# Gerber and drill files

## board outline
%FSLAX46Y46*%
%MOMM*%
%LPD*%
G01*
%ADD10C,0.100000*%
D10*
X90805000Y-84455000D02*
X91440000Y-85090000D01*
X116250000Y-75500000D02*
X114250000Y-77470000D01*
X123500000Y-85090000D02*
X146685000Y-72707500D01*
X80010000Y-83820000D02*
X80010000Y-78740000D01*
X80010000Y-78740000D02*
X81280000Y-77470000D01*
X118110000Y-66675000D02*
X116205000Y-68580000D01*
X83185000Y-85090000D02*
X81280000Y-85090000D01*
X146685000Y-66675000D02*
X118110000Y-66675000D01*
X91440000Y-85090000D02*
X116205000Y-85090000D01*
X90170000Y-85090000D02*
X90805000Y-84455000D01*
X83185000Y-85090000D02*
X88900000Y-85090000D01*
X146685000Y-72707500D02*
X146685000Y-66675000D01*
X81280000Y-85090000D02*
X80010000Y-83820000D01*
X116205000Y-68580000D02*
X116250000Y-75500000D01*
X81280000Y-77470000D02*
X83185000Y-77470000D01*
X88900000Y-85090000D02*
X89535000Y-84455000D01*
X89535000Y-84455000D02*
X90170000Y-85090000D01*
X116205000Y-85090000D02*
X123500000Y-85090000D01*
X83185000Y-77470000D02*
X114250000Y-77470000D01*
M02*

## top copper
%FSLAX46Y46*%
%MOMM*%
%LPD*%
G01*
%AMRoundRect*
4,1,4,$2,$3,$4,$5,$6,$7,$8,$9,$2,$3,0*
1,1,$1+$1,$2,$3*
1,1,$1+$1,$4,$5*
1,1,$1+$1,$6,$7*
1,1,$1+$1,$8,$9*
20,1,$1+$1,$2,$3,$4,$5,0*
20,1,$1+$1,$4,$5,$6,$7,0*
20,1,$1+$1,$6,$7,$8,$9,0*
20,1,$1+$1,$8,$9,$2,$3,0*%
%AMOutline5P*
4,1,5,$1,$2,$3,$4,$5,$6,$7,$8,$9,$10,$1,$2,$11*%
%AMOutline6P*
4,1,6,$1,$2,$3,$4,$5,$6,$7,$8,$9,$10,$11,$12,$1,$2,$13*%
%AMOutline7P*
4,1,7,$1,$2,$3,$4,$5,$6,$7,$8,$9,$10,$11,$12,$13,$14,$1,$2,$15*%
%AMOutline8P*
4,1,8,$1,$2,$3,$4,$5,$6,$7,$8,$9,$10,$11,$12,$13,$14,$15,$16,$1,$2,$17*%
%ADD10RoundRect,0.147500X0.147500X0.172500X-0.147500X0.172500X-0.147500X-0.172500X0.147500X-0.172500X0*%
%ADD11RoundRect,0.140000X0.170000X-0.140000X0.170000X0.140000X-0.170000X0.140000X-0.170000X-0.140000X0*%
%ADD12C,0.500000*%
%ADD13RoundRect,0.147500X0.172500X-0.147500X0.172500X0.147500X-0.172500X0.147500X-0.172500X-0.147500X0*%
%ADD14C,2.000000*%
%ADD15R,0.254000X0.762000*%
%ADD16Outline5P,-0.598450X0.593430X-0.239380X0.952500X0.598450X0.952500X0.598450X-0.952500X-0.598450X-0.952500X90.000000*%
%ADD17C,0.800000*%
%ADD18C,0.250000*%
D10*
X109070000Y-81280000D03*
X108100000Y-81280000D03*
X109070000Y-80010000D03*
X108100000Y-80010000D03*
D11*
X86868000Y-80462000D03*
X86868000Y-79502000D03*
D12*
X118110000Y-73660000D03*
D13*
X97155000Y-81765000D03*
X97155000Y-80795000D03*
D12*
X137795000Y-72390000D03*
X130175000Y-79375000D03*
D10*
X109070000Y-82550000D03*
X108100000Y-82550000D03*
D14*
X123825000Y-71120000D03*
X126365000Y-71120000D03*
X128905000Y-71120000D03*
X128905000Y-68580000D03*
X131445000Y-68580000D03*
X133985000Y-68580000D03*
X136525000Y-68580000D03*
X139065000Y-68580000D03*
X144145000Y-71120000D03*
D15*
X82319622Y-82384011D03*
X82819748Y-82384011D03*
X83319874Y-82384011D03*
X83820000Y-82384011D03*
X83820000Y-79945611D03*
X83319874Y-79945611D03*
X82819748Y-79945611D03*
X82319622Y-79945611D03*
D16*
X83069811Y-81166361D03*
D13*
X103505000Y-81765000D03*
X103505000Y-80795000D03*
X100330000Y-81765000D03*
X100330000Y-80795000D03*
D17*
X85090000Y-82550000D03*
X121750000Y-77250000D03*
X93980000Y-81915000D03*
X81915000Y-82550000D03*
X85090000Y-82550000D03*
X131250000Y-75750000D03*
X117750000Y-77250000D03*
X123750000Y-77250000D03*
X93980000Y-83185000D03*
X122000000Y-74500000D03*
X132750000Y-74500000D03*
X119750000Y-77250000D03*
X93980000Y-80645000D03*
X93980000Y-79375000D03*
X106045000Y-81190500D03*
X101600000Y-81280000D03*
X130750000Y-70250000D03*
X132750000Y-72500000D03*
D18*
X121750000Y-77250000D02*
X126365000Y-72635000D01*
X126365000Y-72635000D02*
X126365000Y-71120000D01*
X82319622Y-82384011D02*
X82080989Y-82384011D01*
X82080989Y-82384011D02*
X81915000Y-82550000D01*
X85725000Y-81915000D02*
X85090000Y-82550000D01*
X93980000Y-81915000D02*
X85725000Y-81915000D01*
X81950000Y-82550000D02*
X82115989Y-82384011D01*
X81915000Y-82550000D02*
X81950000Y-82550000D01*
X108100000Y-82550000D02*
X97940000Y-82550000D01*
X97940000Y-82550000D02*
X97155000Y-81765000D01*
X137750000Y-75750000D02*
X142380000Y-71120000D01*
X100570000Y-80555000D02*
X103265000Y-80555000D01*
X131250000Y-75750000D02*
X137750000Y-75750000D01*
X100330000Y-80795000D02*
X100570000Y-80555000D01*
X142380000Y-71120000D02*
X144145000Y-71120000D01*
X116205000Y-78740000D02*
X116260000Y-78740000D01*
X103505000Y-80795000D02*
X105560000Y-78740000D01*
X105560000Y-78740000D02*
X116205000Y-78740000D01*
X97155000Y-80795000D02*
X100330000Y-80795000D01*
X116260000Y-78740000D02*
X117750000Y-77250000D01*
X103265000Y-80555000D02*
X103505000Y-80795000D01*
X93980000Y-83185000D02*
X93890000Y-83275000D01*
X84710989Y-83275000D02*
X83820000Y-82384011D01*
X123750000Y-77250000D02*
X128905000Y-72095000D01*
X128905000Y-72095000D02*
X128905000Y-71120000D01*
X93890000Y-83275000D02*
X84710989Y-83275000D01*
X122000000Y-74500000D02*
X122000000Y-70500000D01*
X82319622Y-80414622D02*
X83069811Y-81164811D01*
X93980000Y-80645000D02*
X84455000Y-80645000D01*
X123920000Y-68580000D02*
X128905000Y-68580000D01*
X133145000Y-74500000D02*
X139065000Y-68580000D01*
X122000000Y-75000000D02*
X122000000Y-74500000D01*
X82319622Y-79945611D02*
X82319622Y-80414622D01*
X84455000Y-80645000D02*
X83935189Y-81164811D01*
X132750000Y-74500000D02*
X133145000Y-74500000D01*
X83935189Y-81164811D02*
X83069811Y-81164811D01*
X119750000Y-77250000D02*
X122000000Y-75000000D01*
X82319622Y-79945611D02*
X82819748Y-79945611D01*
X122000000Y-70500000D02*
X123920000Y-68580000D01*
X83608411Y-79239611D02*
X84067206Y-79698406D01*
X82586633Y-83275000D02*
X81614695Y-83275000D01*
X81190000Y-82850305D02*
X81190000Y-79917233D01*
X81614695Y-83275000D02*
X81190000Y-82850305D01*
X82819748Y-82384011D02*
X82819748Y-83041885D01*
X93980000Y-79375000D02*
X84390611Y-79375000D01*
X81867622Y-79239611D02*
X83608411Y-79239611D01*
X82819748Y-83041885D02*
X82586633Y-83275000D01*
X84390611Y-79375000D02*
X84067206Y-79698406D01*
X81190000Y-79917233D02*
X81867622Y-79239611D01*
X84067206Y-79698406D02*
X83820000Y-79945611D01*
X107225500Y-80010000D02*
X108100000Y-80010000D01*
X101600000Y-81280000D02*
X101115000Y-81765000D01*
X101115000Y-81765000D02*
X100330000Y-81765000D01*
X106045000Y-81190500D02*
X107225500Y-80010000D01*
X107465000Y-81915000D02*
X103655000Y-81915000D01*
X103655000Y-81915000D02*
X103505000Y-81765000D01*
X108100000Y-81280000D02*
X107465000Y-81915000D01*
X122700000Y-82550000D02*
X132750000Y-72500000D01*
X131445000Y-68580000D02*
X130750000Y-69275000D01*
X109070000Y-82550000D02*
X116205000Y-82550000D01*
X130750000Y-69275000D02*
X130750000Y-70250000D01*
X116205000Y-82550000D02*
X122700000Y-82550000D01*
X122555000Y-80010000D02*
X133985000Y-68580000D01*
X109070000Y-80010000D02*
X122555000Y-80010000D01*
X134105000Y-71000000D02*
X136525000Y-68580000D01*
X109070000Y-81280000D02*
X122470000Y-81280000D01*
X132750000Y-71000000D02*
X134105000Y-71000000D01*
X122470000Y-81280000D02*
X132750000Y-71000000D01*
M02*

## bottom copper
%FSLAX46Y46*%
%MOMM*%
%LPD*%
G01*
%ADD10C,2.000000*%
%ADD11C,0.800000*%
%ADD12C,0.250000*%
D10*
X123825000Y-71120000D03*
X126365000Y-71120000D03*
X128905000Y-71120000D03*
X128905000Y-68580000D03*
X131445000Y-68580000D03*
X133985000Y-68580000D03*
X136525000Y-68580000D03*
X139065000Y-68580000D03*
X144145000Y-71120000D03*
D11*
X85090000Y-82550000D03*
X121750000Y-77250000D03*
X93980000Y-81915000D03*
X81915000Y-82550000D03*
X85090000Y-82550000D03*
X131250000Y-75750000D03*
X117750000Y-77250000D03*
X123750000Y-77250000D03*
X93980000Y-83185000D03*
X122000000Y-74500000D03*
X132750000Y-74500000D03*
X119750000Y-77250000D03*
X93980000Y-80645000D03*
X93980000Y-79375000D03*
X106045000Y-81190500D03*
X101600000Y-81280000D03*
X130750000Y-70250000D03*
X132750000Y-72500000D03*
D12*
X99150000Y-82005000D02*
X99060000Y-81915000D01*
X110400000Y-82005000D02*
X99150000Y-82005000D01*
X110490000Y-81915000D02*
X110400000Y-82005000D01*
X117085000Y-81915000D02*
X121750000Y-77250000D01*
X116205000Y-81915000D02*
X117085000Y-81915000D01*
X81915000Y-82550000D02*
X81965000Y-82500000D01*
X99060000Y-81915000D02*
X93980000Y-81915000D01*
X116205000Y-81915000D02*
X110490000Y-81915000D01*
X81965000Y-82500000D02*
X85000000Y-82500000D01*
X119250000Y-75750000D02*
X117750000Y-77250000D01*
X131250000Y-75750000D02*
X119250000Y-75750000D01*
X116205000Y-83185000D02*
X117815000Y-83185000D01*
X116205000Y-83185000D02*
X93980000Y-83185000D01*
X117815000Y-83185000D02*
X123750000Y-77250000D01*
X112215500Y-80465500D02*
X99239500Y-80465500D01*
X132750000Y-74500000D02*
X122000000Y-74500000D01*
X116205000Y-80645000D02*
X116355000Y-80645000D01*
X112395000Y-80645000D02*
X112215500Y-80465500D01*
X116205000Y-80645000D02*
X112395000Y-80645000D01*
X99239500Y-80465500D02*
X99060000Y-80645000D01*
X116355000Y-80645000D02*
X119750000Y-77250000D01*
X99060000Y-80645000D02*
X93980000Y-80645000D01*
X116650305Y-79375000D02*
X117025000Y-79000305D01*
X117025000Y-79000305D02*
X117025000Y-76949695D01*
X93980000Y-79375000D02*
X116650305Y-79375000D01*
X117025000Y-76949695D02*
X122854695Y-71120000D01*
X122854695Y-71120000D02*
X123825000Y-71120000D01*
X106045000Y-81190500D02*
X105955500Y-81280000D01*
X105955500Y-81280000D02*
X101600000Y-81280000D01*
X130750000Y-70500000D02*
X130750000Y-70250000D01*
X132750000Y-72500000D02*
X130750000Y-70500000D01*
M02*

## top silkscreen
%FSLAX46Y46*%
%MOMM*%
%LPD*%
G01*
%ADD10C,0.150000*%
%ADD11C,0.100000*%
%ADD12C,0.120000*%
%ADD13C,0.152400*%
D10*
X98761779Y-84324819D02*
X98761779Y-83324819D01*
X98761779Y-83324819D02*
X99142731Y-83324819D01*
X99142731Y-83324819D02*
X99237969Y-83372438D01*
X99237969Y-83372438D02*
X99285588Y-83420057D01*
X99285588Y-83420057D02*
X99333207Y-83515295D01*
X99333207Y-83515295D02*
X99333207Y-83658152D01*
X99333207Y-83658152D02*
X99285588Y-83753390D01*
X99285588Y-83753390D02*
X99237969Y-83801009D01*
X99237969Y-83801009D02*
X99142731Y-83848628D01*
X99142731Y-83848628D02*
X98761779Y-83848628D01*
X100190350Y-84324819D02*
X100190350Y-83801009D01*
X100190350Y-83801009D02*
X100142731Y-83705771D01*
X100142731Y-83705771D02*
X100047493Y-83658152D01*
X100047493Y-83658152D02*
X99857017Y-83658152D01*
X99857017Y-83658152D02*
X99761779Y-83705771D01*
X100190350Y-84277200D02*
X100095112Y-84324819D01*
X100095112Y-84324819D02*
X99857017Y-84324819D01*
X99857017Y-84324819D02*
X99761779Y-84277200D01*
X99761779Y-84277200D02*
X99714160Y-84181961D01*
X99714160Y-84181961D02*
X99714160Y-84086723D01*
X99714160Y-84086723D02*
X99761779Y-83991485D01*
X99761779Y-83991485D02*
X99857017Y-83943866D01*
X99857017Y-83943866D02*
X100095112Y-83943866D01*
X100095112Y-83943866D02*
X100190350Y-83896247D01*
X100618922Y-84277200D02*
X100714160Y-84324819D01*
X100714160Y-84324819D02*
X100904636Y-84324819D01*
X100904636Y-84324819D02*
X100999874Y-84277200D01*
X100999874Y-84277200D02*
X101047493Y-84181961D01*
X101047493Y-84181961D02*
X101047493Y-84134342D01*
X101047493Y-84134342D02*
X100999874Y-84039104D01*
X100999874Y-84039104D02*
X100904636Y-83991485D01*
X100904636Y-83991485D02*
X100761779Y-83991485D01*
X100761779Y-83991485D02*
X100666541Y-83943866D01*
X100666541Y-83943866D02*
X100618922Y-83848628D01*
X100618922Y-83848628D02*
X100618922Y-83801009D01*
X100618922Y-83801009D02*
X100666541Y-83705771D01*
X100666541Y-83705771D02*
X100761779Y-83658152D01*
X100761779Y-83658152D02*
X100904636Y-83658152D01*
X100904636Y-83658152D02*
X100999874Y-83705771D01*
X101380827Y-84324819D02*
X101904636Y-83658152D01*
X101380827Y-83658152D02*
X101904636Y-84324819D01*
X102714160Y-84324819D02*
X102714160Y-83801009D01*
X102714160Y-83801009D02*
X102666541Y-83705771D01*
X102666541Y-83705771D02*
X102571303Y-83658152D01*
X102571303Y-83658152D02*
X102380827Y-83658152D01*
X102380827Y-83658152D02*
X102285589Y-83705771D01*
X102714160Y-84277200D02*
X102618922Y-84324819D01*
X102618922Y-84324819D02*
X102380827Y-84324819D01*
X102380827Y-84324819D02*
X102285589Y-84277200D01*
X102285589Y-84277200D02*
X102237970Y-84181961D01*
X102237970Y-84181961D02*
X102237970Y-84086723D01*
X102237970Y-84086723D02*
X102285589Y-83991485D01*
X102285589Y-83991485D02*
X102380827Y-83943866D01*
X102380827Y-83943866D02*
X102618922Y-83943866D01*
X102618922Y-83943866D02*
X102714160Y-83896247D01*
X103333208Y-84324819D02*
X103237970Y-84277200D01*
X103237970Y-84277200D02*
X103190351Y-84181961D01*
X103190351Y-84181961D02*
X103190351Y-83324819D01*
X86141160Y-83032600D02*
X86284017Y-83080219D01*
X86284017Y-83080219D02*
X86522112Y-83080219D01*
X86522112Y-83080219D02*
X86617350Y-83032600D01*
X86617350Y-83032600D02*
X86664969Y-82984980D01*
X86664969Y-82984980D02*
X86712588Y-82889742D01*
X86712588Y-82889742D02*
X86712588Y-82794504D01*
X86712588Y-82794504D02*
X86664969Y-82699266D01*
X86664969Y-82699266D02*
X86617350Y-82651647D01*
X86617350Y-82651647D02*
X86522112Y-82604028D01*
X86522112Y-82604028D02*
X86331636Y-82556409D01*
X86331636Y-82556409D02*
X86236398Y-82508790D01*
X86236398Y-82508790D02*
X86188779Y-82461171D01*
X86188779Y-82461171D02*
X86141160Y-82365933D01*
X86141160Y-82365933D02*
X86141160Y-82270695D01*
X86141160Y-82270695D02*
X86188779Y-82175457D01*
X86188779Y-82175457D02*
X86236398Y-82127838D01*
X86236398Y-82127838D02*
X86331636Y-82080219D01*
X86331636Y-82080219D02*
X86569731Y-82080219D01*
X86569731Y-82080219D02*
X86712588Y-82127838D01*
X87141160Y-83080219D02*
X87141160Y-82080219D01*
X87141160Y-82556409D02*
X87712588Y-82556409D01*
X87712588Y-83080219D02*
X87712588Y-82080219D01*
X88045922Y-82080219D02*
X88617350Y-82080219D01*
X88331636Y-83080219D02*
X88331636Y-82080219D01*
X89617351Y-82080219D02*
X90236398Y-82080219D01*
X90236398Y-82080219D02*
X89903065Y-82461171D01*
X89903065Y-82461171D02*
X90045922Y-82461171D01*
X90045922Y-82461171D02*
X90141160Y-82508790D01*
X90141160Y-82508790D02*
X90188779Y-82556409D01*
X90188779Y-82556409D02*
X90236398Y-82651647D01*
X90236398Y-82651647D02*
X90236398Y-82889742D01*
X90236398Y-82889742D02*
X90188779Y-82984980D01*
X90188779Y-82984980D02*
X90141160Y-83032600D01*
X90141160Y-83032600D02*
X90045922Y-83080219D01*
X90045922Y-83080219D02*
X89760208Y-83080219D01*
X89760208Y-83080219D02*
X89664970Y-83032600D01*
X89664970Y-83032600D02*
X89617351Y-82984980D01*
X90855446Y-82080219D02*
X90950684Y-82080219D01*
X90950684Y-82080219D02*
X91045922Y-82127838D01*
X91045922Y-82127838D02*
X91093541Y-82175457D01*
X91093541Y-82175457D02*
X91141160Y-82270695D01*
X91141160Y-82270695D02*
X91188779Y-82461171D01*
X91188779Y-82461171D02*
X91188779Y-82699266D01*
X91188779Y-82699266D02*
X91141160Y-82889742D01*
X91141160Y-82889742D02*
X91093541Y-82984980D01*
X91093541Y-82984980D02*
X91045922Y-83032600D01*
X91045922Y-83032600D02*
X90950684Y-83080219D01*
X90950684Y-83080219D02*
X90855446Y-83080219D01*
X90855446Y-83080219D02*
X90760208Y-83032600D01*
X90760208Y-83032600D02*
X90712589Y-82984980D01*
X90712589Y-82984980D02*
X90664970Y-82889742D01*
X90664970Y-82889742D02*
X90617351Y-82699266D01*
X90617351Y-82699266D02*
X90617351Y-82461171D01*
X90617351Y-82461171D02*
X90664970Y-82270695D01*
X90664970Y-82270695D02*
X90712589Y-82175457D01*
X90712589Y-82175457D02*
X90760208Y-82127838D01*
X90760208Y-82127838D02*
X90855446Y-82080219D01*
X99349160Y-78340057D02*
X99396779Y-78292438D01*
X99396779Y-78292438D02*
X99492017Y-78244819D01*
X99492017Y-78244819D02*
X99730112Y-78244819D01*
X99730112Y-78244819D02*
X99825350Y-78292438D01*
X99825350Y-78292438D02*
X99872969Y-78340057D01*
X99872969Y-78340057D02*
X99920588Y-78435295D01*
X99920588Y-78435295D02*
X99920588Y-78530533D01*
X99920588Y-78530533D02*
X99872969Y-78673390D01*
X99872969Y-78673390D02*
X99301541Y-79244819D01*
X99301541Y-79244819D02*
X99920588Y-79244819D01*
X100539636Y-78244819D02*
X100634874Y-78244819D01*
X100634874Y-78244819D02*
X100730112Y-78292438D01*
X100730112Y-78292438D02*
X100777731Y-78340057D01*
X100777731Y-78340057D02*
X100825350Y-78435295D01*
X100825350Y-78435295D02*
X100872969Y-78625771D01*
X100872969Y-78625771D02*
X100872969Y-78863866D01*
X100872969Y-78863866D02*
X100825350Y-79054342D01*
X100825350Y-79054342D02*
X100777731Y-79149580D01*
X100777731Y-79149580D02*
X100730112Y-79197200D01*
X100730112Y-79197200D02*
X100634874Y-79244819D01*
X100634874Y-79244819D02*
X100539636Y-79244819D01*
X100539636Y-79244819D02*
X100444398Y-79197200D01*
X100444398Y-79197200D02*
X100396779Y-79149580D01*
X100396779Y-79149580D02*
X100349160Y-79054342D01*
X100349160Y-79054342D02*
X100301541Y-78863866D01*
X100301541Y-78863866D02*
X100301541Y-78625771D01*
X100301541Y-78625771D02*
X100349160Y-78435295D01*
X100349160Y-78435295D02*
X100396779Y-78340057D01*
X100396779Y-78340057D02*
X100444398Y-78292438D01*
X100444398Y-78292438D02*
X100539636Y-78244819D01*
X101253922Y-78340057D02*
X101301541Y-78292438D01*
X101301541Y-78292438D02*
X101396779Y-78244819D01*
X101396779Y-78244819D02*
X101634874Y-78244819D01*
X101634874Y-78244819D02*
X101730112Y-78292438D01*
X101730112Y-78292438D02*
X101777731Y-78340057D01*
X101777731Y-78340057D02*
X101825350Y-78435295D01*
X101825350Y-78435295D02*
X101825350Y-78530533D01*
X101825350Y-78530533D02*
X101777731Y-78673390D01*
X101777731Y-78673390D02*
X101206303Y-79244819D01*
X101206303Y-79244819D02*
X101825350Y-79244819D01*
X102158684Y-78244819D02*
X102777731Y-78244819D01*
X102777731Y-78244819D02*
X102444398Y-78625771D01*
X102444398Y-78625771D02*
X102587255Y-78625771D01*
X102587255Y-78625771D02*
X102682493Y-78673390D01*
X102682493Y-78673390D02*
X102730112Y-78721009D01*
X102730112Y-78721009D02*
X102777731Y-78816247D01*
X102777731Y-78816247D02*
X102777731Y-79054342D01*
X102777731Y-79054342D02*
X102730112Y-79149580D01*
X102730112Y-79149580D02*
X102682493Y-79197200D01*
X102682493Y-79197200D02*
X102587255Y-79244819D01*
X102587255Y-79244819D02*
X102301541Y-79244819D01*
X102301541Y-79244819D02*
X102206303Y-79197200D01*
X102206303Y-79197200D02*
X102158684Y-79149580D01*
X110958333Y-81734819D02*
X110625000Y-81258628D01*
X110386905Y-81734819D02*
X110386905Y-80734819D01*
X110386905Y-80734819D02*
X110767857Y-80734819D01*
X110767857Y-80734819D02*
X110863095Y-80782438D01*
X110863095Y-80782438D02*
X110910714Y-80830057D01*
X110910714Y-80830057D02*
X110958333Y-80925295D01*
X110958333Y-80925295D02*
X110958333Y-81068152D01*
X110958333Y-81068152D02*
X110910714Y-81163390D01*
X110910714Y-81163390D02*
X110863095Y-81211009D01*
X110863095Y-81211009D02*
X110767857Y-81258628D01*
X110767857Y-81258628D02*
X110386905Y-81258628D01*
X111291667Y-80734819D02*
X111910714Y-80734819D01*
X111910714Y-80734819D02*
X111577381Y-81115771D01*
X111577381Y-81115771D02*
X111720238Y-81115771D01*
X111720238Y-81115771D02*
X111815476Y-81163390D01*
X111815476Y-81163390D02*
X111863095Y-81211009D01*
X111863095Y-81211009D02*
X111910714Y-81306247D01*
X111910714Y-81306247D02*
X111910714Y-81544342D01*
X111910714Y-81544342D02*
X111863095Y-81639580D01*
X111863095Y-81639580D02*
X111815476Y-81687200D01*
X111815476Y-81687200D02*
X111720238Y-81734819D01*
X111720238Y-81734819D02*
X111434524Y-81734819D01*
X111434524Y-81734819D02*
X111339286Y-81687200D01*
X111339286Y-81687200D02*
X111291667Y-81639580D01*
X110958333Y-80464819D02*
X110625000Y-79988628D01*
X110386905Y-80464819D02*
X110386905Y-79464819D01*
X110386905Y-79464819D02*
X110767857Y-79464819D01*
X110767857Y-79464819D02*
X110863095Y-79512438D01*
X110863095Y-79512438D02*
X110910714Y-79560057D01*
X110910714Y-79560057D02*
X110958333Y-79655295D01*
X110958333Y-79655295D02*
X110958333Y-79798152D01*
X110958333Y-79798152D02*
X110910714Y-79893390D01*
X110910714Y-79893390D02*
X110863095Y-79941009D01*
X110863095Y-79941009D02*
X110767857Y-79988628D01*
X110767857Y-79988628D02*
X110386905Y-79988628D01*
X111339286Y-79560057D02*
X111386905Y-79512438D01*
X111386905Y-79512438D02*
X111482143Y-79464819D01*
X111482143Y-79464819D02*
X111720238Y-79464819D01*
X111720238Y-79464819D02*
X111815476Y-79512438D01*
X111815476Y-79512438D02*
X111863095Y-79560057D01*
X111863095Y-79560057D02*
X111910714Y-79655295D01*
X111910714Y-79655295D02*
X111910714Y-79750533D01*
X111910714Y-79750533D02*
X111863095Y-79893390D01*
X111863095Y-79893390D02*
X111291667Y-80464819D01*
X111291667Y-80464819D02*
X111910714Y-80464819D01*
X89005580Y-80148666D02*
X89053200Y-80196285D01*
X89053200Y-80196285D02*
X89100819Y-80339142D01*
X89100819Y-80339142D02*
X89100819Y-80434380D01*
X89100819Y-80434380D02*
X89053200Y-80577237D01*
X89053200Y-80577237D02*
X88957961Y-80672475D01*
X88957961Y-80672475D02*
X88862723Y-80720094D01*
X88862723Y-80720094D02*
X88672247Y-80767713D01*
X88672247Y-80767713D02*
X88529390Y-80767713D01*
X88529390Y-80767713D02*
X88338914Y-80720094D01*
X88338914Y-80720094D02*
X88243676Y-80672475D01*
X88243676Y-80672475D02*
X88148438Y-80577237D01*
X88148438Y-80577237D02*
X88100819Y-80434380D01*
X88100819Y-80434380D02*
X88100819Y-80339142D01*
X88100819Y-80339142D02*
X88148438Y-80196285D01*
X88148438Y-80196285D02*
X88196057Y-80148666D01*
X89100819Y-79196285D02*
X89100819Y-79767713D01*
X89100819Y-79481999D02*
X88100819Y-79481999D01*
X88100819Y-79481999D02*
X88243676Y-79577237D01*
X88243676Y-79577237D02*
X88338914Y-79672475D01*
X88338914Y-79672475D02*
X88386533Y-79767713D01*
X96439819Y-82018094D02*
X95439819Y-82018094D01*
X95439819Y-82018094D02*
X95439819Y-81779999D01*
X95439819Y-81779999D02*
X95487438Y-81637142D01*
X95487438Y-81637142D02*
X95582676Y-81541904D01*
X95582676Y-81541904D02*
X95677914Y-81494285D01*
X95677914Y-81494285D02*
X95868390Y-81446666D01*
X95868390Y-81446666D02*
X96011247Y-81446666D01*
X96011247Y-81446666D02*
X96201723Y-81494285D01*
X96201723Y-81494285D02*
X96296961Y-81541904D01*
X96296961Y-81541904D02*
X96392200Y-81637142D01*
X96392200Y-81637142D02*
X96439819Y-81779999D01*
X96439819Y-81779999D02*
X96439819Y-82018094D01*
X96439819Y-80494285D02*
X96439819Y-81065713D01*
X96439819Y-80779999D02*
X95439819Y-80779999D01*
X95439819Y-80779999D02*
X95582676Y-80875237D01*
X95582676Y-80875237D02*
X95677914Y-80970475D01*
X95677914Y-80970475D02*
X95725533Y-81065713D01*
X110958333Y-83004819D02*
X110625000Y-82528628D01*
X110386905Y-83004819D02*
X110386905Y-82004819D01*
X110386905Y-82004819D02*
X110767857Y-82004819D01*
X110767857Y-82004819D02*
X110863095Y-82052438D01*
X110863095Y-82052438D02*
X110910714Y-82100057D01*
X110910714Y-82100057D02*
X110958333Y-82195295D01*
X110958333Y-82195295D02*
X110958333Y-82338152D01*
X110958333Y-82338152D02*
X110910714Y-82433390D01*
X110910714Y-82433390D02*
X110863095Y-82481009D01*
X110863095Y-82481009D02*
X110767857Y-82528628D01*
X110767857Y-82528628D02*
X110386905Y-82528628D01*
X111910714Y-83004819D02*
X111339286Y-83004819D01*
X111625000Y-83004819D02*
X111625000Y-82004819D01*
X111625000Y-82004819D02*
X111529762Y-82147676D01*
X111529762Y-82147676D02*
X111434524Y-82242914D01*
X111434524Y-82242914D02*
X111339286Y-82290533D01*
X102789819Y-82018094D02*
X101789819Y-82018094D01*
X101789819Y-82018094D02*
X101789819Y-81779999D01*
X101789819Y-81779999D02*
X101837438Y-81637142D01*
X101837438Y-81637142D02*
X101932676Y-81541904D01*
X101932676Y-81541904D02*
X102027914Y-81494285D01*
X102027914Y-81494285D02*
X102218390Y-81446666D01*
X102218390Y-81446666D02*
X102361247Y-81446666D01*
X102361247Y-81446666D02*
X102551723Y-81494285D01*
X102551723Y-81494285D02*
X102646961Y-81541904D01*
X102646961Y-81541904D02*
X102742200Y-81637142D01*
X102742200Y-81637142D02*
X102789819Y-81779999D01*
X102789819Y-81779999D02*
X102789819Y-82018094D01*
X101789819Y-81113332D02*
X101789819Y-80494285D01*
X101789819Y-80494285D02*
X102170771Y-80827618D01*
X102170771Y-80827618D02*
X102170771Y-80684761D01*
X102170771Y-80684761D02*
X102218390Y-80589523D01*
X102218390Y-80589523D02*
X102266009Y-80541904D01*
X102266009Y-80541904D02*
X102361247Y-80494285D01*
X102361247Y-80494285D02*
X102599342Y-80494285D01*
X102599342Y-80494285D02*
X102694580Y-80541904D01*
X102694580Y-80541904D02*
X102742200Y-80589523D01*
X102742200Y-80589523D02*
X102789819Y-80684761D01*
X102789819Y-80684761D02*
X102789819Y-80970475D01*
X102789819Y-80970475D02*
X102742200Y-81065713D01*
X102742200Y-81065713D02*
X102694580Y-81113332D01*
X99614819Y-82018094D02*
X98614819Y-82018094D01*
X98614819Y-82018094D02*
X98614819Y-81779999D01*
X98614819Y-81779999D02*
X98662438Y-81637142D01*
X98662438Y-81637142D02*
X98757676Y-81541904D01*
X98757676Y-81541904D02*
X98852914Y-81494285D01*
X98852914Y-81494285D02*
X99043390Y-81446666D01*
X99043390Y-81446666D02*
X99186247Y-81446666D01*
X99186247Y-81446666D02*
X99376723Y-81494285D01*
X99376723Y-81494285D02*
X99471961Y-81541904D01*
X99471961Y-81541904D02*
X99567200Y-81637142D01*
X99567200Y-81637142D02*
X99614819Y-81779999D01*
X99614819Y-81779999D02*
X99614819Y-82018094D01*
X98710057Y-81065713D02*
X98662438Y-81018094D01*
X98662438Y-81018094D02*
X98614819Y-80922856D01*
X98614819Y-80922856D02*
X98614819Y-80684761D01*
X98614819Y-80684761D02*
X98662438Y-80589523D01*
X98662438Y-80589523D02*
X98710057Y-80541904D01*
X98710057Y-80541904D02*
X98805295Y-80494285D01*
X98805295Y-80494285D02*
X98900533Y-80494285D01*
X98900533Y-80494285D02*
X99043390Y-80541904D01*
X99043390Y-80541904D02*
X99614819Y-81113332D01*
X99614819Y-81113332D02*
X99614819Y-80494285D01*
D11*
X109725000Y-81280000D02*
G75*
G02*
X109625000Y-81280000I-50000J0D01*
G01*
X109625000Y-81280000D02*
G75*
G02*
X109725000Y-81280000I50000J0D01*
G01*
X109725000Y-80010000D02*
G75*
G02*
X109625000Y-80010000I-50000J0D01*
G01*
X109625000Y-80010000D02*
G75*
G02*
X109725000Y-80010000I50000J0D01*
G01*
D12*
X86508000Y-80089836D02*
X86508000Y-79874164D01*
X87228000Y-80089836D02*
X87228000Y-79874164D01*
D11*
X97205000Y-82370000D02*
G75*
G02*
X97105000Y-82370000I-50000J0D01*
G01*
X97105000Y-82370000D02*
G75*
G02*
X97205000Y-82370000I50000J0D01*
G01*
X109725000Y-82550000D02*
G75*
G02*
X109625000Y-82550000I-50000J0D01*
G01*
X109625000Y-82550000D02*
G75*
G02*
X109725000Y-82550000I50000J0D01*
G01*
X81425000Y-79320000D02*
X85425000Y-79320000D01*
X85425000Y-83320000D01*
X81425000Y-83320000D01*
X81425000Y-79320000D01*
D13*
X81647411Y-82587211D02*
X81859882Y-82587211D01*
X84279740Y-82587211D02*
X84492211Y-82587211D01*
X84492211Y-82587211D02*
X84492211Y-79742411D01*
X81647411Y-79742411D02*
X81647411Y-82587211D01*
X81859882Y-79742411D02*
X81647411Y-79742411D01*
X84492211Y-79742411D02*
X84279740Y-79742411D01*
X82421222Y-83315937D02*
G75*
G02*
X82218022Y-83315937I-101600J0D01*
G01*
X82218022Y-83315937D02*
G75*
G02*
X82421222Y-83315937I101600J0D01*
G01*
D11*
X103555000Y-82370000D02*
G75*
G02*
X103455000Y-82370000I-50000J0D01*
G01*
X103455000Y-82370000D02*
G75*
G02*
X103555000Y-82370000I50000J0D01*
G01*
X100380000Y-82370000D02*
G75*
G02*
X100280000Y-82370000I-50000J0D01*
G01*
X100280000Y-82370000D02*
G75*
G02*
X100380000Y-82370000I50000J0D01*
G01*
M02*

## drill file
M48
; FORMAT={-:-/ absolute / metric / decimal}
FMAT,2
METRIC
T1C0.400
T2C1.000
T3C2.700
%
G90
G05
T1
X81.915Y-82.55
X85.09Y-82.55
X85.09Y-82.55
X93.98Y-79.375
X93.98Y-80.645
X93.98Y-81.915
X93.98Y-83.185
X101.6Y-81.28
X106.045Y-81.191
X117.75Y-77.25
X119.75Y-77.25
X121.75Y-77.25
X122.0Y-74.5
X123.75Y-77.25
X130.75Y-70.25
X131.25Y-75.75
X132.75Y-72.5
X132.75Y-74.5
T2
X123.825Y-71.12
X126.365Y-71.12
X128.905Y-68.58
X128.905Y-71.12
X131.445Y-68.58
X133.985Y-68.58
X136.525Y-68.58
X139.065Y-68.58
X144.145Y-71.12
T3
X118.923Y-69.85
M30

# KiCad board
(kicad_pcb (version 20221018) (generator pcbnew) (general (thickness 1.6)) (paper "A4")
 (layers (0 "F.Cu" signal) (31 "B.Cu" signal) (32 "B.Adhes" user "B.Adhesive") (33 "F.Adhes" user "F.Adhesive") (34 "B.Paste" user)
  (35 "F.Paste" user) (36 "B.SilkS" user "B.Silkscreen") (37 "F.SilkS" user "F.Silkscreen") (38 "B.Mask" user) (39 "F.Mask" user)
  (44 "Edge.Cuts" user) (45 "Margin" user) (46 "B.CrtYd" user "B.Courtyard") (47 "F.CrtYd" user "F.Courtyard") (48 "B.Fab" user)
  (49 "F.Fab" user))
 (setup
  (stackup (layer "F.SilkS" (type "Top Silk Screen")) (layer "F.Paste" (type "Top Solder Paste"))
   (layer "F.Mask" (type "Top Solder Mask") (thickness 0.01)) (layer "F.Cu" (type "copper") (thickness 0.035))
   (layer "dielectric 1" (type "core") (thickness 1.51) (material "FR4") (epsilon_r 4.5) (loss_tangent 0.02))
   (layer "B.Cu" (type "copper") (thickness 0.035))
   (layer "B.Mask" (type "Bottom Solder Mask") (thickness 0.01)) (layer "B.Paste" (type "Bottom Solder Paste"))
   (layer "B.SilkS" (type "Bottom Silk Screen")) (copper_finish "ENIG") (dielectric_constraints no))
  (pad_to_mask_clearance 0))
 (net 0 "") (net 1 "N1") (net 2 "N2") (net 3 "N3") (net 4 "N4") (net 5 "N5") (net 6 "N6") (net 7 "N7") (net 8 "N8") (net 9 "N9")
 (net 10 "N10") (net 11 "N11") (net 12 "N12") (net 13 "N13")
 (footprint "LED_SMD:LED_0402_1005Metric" (layer "F.Cu") (at 108.585 81.28 180)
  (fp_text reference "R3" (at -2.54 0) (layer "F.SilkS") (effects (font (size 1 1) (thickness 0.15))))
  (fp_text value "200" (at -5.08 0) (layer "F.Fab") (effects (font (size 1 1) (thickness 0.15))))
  (fp_circle (center -1.09 0) (end -1.04 0) (stroke (width 0.1) (type solid)) (fill none) (layer "F.SilkS"))
  (pad "1" smd roundrect (at -0.485 0 180) (size 0.59 0.64) (layers "F.Cu" "F.Paste" "F.Mask") (roundrect_rratio 0.25) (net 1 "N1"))
  (pad "2" smd roundrect (at 0.485 0 180) (size 0.59 0.64) (layers "F.Cu" "F.Paste" "F.Mask") (roundrect_rratio 0.25) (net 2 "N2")))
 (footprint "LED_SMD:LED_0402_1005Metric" (layer "F.Cu") (at 108.585 80.01 180)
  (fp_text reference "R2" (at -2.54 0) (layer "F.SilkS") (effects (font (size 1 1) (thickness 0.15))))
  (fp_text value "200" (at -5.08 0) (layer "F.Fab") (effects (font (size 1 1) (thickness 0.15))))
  (fp_circle (center -1.09 0) (end -1.04 0) (stroke (width 0.1) (type solid)) (fill none) (layer "F.SilkS"))
  (pad "1" smd roundrect (at -0.485 0 180) (size 0.59 0.64) (layers "F.Cu" "F.Paste" "F.Mask") (roundrect_rratio 0.25) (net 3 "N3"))
  (pad "2" smd roundrect (at 0.485 0 180) (size 0.59 0.64) (layers "F.Cu" "F.Paste" "F.Mask") (roundrect_rratio 0.25) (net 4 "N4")))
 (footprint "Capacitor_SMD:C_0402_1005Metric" (layer "F.Cu") (at 86.868 79.982 90)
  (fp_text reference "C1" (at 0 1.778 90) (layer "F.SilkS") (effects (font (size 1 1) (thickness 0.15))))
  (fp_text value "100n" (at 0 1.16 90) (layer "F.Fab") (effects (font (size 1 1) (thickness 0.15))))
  (fp_line (start -0.107836 -0.36) (end 0.107836 -0.36) (stroke (width 0.12) (type solid)) (layer "F.SilkS"))
  (fp_line (start -0.107836 0.36) (end 0.107836 0.36) (stroke (width 0.12) (type solid)) (layer "F.SilkS"))
  (pad "1" smd roundrect (at -0.48 0 90) (size 0.56 0.62) (layers "F.Cu" "F.Paste" "F.Mask") (roundrect_rratio 0.25) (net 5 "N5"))
  (pad "2" smd roundrect (at 0.48 0 90) (size 0.56 0.62) (layers "F.Cu" "F.Paste" "F.Mask") (roundrect_rratio 0.25) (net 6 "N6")))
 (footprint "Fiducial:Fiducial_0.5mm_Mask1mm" (layer "F.Cu") (at 118.11 73.66)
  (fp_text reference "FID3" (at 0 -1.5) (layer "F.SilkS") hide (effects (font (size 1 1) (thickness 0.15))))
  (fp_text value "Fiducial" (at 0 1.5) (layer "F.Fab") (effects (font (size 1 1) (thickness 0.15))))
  (pad "" smd circle (at 0 0) (size 0.5 0.5) (layers "F.Cu" "F.Mask") (solder_mask_margin 0.25) (clearance 0.25)))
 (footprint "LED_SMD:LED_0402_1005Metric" (layer "F.Cu") (at 97.155 81.28 90)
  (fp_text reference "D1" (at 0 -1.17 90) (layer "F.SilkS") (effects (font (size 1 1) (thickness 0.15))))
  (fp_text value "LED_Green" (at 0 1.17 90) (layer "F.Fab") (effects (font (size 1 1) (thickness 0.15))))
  (fp_circle (center -1.09 0) (end -1.04 0) (stroke (width 0.1) (type solid)) (fill none) (layer "F.SilkS"))
  (pad "1" smd roundrect (at -0.485 0 90) (size 0.59 0.64) (layers "F.Cu" "F.Paste" "F.Mask") (roundrect_rratio 0.25) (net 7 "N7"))
  (pad "2" smd roundrect (at 0.485 0 90) (size 0.59 0.64) (layers "F.Cu" "F.Paste" "F.Mask") (roundrect_rratio 0.25) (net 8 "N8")))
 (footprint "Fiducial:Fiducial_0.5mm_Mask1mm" (layer "F.Cu") (at 137.795 72.39)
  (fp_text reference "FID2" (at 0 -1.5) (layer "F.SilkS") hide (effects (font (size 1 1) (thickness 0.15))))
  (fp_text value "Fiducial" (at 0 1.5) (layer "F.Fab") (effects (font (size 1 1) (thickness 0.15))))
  (pad "" smd circle (at 0 0) (size 0.5 0.5) (layers "F.Cu" "F.Mask") (solder_mask_margin 0.25) (clearance 0.25)))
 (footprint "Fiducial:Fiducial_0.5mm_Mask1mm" (layer "F.Cu") (at 130.175 79.375)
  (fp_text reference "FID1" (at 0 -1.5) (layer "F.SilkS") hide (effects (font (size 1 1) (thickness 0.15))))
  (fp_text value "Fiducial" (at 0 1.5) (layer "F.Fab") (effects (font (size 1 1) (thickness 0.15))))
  (pad "" smd circle (at 0 0) (size 0.5 0.5) (layers "F.Cu" "F.Mask") (solder_mask_margin 0.25) (clearance 0.25)))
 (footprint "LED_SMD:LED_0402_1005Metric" (layer "F.Cu") (at 108.585 82.55 180)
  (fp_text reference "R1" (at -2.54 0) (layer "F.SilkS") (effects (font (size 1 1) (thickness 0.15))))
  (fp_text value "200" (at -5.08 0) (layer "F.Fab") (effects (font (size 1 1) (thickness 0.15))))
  (fp_circle (center -1.09 0) (end -1.04 0) (stroke (width 0.1) (type solid)) (fill none) (layer "F.SilkS"))
  (pad "1" smd roundrect (at -0.485 0 180) (size 0.59 0.64) (layers "F.Cu" "F.Paste" "F.Mask") (roundrect_rratio 0.25) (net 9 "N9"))
  (pad "2" smd roundrect (at 0.485 0 180) (size 0.59 0.64) (layers "F.Cu" "F.Paste" "F.Mask") (roundrect_rratio 0.25) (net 7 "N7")))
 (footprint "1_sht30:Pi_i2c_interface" (layer "F.Cu") (at 123.825 71.12)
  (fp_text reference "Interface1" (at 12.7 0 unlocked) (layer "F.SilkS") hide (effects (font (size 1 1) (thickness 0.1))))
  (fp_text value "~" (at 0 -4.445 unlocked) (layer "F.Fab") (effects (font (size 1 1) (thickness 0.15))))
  (fp_rect (start -42.4 8.2) (end -38.4 12.2) (stroke (width 0.1) (type default)) (fill none) (layer "F.SilkS"))
  (pad "1" thru_hole circle (at 0 0) (size 2 2) (drill 1) (layers "*.Cu" "*.Mask") (remove_unused_layers) (keep_end_layers)
   (zone_layer_connections) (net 6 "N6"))
  (pad "2" thru_hole circle (at 2.54 0) (size 2 2) (drill 1) (layers "*.Cu" "*.Mask") (remove_unused_layers) (keep_end_layers)
   (zone_layer_connections) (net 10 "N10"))
  (pad "3" thru_hole circle (at 5.08 0) (size 2 2) (drill 1) (layers "*.Cu" "*.Mask") (remove_unused_layers) (keep_end_layers)
   (zone_layer_connections) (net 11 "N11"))
  (pad "4" thru_hole circle (at 5.08 -2.54) (size 2 2) (drill 1) (layers "*.Cu" "*.Mask") (remove_unused_layers) (keep_end_layers)
   (zone_layer_connections) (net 5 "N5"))
  (pad "5" thru_hole circle (at 7.62 -2.54) (size 2 2) (drill 1) (layers "*.Cu" "*.Mask") (remove_unused_layers) (keep_end_layers)
   (zone_layer_connections) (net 9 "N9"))
  (pad "6" thru_hole circle (at 10.16 -2.54) (size 2 2) (drill 1) (layers "*.Cu" "*.Mask") (remove_unused_layers) (keep_end_layers)
   (zone_layer_connections) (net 3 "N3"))
  (pad "7" thru_hole circle (at 12.7 -2.54) (size 2 2) (drill 1) (layers "*.Cu" "*.Mask") (remove_unused_layers) (keep_end_layers)
   (zone_layer_connections) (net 1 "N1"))
  (pad "8" thru_hole circle (at 15.24 -2.54) (size 2 2) (drill 1) (layers "*.Cu" "*.Mask") (remove_unused_layers) (keep_end_layers)
   (zone_layer_connections) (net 5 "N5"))
  (pad "9" thru_hole circle (at 20.32 0) (size 2 2) (drill 1) (layers "*.Cu" "*.Mask") (remove_unused_layers) (keep_end_layers)
   (zone_layer_connections) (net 8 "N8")))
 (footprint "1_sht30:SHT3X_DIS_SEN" (layer "F.Cu") (at 83.069811 81.164811 90)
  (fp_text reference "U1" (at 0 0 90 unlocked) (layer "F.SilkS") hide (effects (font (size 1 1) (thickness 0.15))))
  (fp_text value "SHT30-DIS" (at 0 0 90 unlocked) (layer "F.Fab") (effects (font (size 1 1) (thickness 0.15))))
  (fp_line (start -1.4224 -1.4224) (end -1.4224 -1.209929) (stroke (width 0.1524) (type solid)) (layer "F.SilkS"))
  (fp_line (start -1.4224 1.209929) (end -1.4224 1.4224) (stroke (width 0.1524) (type solid)) (layer "F.SilkS"))
  (fp_line (start -1.4224 1.4224) (end 1.4224 1.4224) (stroke (width 0.1524) (type solid)) (layer "F.SilkS"))
  (fp_line (start 1.4224 -1.4224) (end -1.4224 -1.4224) (stroke (width 0.1524) (type solid)) (layer "F.SilkS"))
  (fp_line (start 1.4224 -1.209929) (end 1.4224 -1.4224) (stroke (width 0.1524) (type solid)) (layer "F.SilkS"))
  (fp_line (start 1.4224 1.4224) (end 1.4224 1.209929) (stroke (width 0.1524) (type solid)) (layer "F.SilkS"))
  (fp_circle (center -2.151126 -0.750189) (end -2.049526 -0.750189) (stroke (width 0.1524) (type solid)) (fill none) (layer "F.SilkS"))
  (pad "1" smd rect (at -1.2192 -0.750189 90) (size 0.762 0.254) (layers "F.Cu" "F.Paste" "F.Mask") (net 10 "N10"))
  (pad "2" smd rect (at -1.2192 -0.250063 90) (size 0.762 0.254) (layers "F.Cu" "F.Paste" "F.Mask") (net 6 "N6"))
  (pad "3" smd rect (at -1.2192 0.250063 90) (size 0.762 0.254) (layers "F.Cu" "F.Paste" "F.Mask") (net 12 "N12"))
  (pad "4" smd rect (at -1.2192 0.750189 90) (size 0.762 0.254) (layers "F.Cu" "F.Paste" "F.Mask") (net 11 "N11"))
  (pad "5" smd rect (at 1.2192 0.750189 90) (size 0.762 0.254) (layers "F.Cu" "F.Paste" "F.Mask") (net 6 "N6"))
  (pad "6" smd rect (at 1.2192 0.250063 90) (size 0.762 0.254) (layers "F.Cu" "F.Paste" "F.Mask") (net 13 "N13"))
  (pad "7" smd rect (at 1.2192 -0.250063 90) (size 0.762 0.254) (layers "F.Cu" "F.Paste" "F.Mask") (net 5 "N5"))
  (pad "8" smd rect (at 1.2192 -0.750189 90) (size 0.762 0.254) (layers "F.Cu" "F.Paste" "F.Mask") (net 5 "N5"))
  (pad "9" smd roundrect (at -0.00155 0 90) (size 1.1969 1.905) (layers "F.Cu" "F.Paste" "F.Mask") (roundrect_rratio 0) (chamfer_ratio 0.3)
   (chamfer top_left) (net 5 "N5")))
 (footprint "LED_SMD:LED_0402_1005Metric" (layer "F.Cu") (at 103.505 81.28 90)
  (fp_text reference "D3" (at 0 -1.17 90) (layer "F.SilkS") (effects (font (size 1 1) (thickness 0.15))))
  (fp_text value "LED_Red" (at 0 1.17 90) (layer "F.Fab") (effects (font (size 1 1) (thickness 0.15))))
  (fp_circle (center -1.09 0) (end -1.04 0) (stroke (width 0.1) (type solid)) (fill none) (layer "F.SilkS"))
  (pad "1" smd roundrect (at -0.485 0 90) (size 0.59 0.64) (layers "F.Cu" "F.Paste" "F.Mask") (roundrect_rratio 0.25) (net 2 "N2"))
  (pad "2" smd roundrect (at 0.485 0 90) (size 0.59 0.64) (layers "F.Cu" "F.Paste" "F.Mask") (roundrect_rratio 0.25) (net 8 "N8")))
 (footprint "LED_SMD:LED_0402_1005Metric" (layer "F.Cu") (at 100.33 81.28 90)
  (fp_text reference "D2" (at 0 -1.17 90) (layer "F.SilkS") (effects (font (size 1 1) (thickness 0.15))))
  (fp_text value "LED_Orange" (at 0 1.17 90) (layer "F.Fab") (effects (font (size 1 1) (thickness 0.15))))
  (fp_circle (center -1.09 0) (end -1.04 0) (stroke (width 0.1) (type solid)) (fill none) (layer "F.SilkS"))
  (pad "1" smd roundrect (at -0.485 0 90) (size 0.59 0.64) (layers "F.Cu" "F.Paste" "F.Mask") (roundrect_rratio 0.25) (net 4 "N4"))
  (pad "2" smd roundrect (at 0.485 0 90) (size 0.59 0.64) (layers "F.Cu" "F.Paste" "F.Mask") (roundrect_rratio 0.25) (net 8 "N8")))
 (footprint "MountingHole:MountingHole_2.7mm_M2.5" (layer "F.Cu") (at 118.9228 69.85)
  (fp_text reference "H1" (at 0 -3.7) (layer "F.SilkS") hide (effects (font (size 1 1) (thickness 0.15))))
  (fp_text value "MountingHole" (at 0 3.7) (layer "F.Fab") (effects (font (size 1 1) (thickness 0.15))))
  (pad "" np_thru_hole circle (at 0 0) (size 2.7 2.7) (drill 2.7) (layers "*.Cu" "*.Mask")))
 (gr_line (start 90.805 84.455) (end 91.44 85.09) (stroke (width 0.1) (type default)) (layer "Edge.Cuts"))
 (gr_line (start 116.25 75.5) (end 114.25 77.47) (stroke (width 0.1) (type default)) (layer "Edge.Cuts"))
 (gr_line (start 123.5 85.09) (end 146.685 72.7075) (stroke (width 0.1) (type default)) (layer "Edge.Cuts"))
 (gr_line (start 80.01 83.82) (end 80.01 78.74) (stroke (width 0.1) (type default)) (layer "Edge.Cuts"))
 (gr_line (start 80.01 78.74) (end 81.28 77.47) (stroke (width 0.1) (type default)) (layer "Edge.Cuts"))
 (gr_line (start 118.11 66.675) (end 116.205 68.58) (stroke (width 0.1) (type default)) (layer "Edge.Cuts"))
 (gr_line (start 83.185 85.09) (end 81.28 85.09) (stroke (width 0.1) (type default)) (layer "Edge.Cuts"))
 (gr_line (start 146.685 66.675) (end 118.11 66.675) (stroke (width 0.1) (type default)) (layer "Edge.Cuts"))
 (gr_line (start 91.44 85.09) (end 116.205 85.09) (stroke (width 0.1) (type default)) (layer "Edge.Cuts"))
 (gr_line (start 90.17 85.09) (end 90.805 84.455) (stroke (width 0.1) (type default)) (layer "Edge.Cuts"))
 (gr_line (start 83.185 85.09) (end 88.9 85.09) (stroke (width 0.1) (type default)) (layer "Edge.Cuts"))
 (gr_line (start 146.685 72.7075) (end 146.685 66.675) (stroke (width 0.1) (type default)) (layer "Edge.Cuts"))
 (gr_line (start 81.28 85.09) (end 80.01 83.82) (stroke (width 0.1) (type default)) (layer "Edge.Cuts"))
 (gr_line (start 116.205 68.58) (end 116.25 75.5) (stroke (width 0.1) (type default)) (layer "Edge.Cuts"))
 (gr_line (start 81.28 77.47) (end 83.185 77.47) (stroke (width 0.1) (type default)) (layer "Edge.Cuts"))
 (gr_line (start 88.9 85.09) (end 89.535 84.455) (stroke (width 0.1) (type default)) (layer "Edge.Cuts"))
 (gr_line (start 89.535 84.455) (end 90.17 85.09) (stroke (width 0.1) (type default)) (layer "Edge.Cuts"))
 (gr_line (start 116.205 85.09) (end 123.5 85.09) (stroke (width 0.1) (type default)) (layer "Edge.Cuts"))
 (gr_line (start 83.185 77.47) (end 114.25 77.47) (stroke (width 0.1) (type default)) (layer "Edge.Cuts"))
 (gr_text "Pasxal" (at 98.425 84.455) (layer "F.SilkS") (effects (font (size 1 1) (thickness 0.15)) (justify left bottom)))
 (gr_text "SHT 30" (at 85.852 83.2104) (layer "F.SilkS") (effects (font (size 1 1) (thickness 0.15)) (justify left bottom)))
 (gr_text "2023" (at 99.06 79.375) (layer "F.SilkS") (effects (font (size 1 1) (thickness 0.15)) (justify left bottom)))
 (segment (start 121.75 77.25) (end 126.365 72.635) (width 0.25) (layer "F.Cu") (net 10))
 (segment (start 126.365 72.635) (end 126.365 71.12) (width 0.25) (layer "F.Cu") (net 10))
 (segment (start 82.319622 82.384011) (end 82.080989 82.384011) (width 0.25) (layer "F.Cu") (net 10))
 (segment (start 82.080989 82.384011) (end 81.915 82.55) (width 0.25) (layer "F.Cu") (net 10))
 (segment (start 85.725 81.915) (end 85.09 82.55) (width 0.25) (layer "F.Cu") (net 10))
 (segment (start 93.98 81.915) (end 85.725 81.915) (width 0.25) (layer "F.Cu") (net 10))
 (segment (start 81.95 82.55) (end 82.115989 82.384011) (width 0.25) (layer "F.Cu") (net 10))
 (segment (start 81.915 82.55) (end 81.95 82.55) (width 0.25) (layer "F.Cu") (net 10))
 (via (at 85.09 82.55) (size 0.8) (drill 0.4) (layers "F.Cu" "B.Cu") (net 10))
 (via (at 121.75 77.25) (size 0.8) (drill 0.4) (layers "F.Cu" "B.Cu") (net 10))
 (via (at 93.98 81.915) (size 0.8) (drill 0.4) (layers "F.Cu" "B.Cu") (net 10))
 (via (at 81.915 82.55) (size 0.8) (drill 0.4) (layers "F.Cu" "B.Cu") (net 10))
 (via (at 85.09 82.55) (size 0.8) (drill 0.4) (layers "F.Cu" "B.Cu") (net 10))
 (segment (start 99.15 82.005) (end 99.06 81.915) (width 0.25) (layer "B.Cu") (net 10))
 (segment (start 110.4 82.005) (end 99.15 82.005) (width 0.25) (layer "B.Cu") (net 10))
 (segment (start 110.49 81.915) (end 110.4 82.005) (width 0.25) (layer "B.Cu") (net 10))
 (segment (start 117.085 81.915) (end 121.75 77.25) (width 0.25) (layer "B.Cu") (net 10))
 (segment (start 116.205 81.915) (end 117.085 81.915) (width 0.25) (layer "B.Cu") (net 10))
 (segment (start 81.915 82.55) (end 81.965 82.5) (width 0.25) (layer "B.Cu") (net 10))
 (segment (start 99.06 81.915) (end 93.98 81.915) (width 0.25) (layer "B.Cu") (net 10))
 (segment (start 116.205 81.915) (end 110.49 81.915) (width 0.25) (layer "B.Cu") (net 10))
 (segment (start 81.965 82.5) (end 85 82.5) (width 0.25) (layer "B.Cu") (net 10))
 (segment (start 108.1 82.55) (end 97.94 82.55) (width 0.25) (layer "F.Cu") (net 7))
 (segment (start 97.94 82.55) (end 97.155 81.765) (width 0.25) (layer "F.Cu") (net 7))
 (segment (start 137.75 75.75) (end 142.38 71.12) (width 0.25) (layer "F.Cu") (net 8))
 (segment (start 100.57 80.555) (end 103.265 80.555) (width 0.25) (layer "F.Cu") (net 8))
 (segment (start 131.25 75.75) (end 137.75 75.75) (width 0.25) (layer "F.Cu") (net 8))
 (segment (start 100.33 80.795) (end 100.57 80.555) (width 0.25) (layer "F.Cu") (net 8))
 (segment (start 142.38 71.12) (end 144.145 71.12) (width 0.25) (layer "F.Cu") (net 8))
 (segment (start 116.205 78.74) (end 116.26 78.74) (width 0.25) (layer "F.Cu") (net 8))
 (segment (start 103.505 80.795) (end 105.56 78.74) (width 0.25) (layer "F.Cu") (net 8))
 (segment (start 105.56 78.74) (end 116.205 78.74) (width 0.25) (layer "F.Cu") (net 8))
 (segment (start 97.155 80.795) (end 100.33 80.795) (width 0.25) (layer "F.Cu") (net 8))
 (segment (start 116.26 78.74) (end 117.75 77.25) (width 0.25) (layer "F.Cu") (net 8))
 (segment (start 103.265 80.555) (end 103.505 80.795) (width 0.25) (layer "F.Cu") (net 8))
 (via (at 131.25 75.75) (size 0.8) (drill 0.4) (layers "F.Cu" "B.Cu") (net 8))
 (via (at 117.75 77.25) (size 0.8) (drill 0.4) (layers "F.Cu" "B.Cu") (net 8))
 (segment (start 119.25 75.75) (end 117.75 77.25) (width 0.25) (layer "B.Cu") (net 8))
 (segment (start 131.25 75.75) (end 119.25 75.75) (width 0.25) (layer "B.Cu") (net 8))
 (segment (start 93.98 83.185) (end 93.89 83.275) (width 0.25) (layer "F.Cu") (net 11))
 (segment (start 84.710989 83.275) (end 83.82 82.384011) (width 0.25) (layer "F.Cu") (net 11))
 (segment (start 123.75 77.25) (end 128.905 72.095) (width 0.25) (layer "F.Cu") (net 11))
 (segment (start 128.905 72.095) (end 128.905 71.12) (width 0.25) (layer "F.Cu") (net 11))
 (segment (start 93.89 83.275) (end 84.710989 83.275) (width 0.25) (layer "F.Cu") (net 11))
 (via (at 123.75 77.25) (size 0.8) (drill 0.4) (layers "F.Cu" "B.Cu") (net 11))
 (via (at 93.98 83.185) (size 0.8) (drill 0.4) (layers "F.Cu" "B.Cu") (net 11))
 (segment (start 116.205 83.185) (end 117.815 83.185) (width 0.25) (layer "B.Cu") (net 11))
 (segment (start 116.205 83.185) (end 93.98 83.185) (width 0.25) (layer "B.Cu") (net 11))
 (segment (start 117.815 83.185) (end 123.75 77.25) (width 0.25) (layer "B.Cu") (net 11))
 (segment (start 122 74.5) (end 122 70.5) (width 0.25) (layer "F.Cu") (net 5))
 (segment (start 82.319622 80.414622) (end 83.069811 81.164811) (width 0.25) (layer "F.Cu") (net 5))
 (segment (start 93.98 80.645) (end 84.455 80.645) (width 0.25) (layer "F.Cu") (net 5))
 (segment (start 123.92 68.58) (end 128.905 68.58) (width 0.25) (layer "F.Cu") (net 5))
 (segment (start 133.145 74.5) (end 139.065 68.58) (width 0.25) (layer "F.Cu") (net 5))
 (segment (start 122 75) (end 122 74.5) (width 0.25) (layer "F.Cu") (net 5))
 (segment (start 82.319622 79.945611) (end 82.319622 80.414622) (width 0.25) (layer "F.Cu") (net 5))
 (segment (start 84.455 80.645) (end 83.935189 81.164811) (width 0.25) (layer "F.Cu") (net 5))
 (segment (start 132.75 74.5) (end 133.145 74.5) (width 0.25) (layer "F.Cu") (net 5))
 (segment (start 83.935189 81.164811) (end 83.069811 81.164811) (width 0.25) (layer "F.Cu") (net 5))
 (segment (start 119.75 77.25) (end 122 75) (width 0.25) (layer "F.Cu") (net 5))
 (segment (start 82.319622 79.945611) (end 82.819748 79.945611) (width 0.25) (layer "F.Cu") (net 5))
 (segment (start 122 70.5) (end 123.92 68.58) (width 0.25) (layer "F.Cu") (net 5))
 (via (at 122 74.5) (size 0.8) (drill 0.4) (layers "F.Cu" "B.Cu") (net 5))
 (via (at 132.75 74.5) (size 0.8) (drill 0.4) (layers "F.Cu" "B.Cu") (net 5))
 (via (at 119.75 77.25) (size 0.8) (drill 0.4) (layers "F.Cu" "B.Cu") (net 5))
 (via (at 93.98 80.645) (size 0.8) (drill 0.4) (layers "F.Cu" "B.Cu") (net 5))
 (segment (start 112.2155 80.4655) (end 99.2395 80.4655) (width 0.25) (layer "B.Cu") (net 5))
 (segment (start 132.75 74.5) (end 122 74.5) (width 0.25) (layer "B.Cu") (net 5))
 (segment (start 116.205 80.645) (end 116.355 80.645) (width 0.25) (layer "B.Cu") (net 5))
 (segment (start 112.395 80.645) (end 112.2155 80.4655) (width 0.25) (layer "B.Cu") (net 5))
 (segment (start 116.205 80.645) (end 112.395 80.645) (width 0.25) (layer "B.Cu") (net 5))
 (segment (start 99.2395 80.4655) (end 99.06 80.645) (width 0.25) (layer "B.Cu") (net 5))
 (segment (start 116.355 80.645) (end 119.75 77.25) (width 0.25) (layer "B.Cu") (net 5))
 (segment (start 99.06 80.645) (end 93.98 80.645) (width 0.25) (layer "B.Cu") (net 5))
 (segment (start 83.608411 79.239611) (end 84.067206 79.698406) (width 0.25) (layer "F.Cu") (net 6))
 (segment (start 82.586633 83.275) (end 81.614695 83.275) (width 0.25) (layer "F.Cu") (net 6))
 (segment (start 81.19 82.850305) (end 81.19 79.917233) (width 0.25) (layer "F.Cu") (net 6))
 (segment (start 81.614695 83.275) (end 81.19 82.850305) (width 0.25) (layer "F.Cu") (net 6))
 (segment (start 82.819748 82.384011) (end 82.819748 83.041885) (width 0.25) (layer "F.Cu") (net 6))
 (segment (start 93.98 79.375) (end 84.390611 79.375) (width 0.25) (layer "F.Cu") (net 6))
 (segment (start 81.867622 79.239611) (end 83.608411 79.239611) (width 0.25) (layer "F.Cu") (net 6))
 (segment (start 82.819748 83.041885) (end 82.586633 83.275) (width 0.25) (layer "F.Cu") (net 6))
 (segment (start 84.390611 79.375) (end 84.067206 79.698406) (width 0.25) (layer "F.Cu") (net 6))
 (segment (start 81.19 79.917233) (end 81.867622 79.239611) (width 0.25) (layer "F.Cu") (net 6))
 (segment (start 84.067206 79.698406) (end 83.82 79.945611) (width 0.25) (layer "F.Cu") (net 6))
 (via (at 93.98 79.375) (size 0.8) (drill 0.4) (layers "F.Cu" "B.Cu") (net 6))
 (segment (start 116.650305 79.375) (end 117.025 79.000305) (width 0.25) (layer "B.Cu") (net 6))
 (segment (start 117.025 79.000305) (end 117.025 76.949695) (width 0.25) (layer "B.Cu") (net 6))
 (segment (start 93.98 79.375) (end 116.650305 79.375) (width 0.25) (layer "B.Cu") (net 6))
 (segment (start 117.025 76.949695) (end 122.854695 71.12) (width 0.25) (layer "B.Cu") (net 6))
 (segment (start 122.854695 71.12) (end 123.825 71.12) (width 0.25) (layer "B.Cu") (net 6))
 (segment (start 107.2255 80.01) (end 108.1 80.01) (width 0.25) (layer "F.Cu") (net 4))
 (segment (start 101.6 81.28) (end 101.115 81.765) (width 0.25) (layer "F.Cu") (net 4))
 (segment (start 101.115 81.765) (end 100.33 81.765) (width 0.25) (layer "F.Cu") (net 4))
 (segment (start 106.045 81.1905) (end 107.2255 80.01) (width 0.25) (layer "F.Cu") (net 4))
 (via (at 106.045 81.1905) (size 0.8) (drill 0.4) (layers "F.Cu" "B.Cu") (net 4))
 (via (at 101.6 81.28) (size 0.8) (drill 0.4) (layers "F.Cu" "B.Cu") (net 4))
 (segment (start 106.045 81.1905) (end 105.9555 81.28) (width 0.25) (layer "B.Cu") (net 4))
 (segment (start 105.9555 81.28) (end 101.6 81.28) (width 0.25) (layer "B.Cu") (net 4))
 (segment (start 107.465 81.915) (end 103.655 81.915) (width 0.25) (layer "F.Cu") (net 2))
 (segment (start 103.655 81.915) (end 103.505 81.765) (width 0.25) (layer "F.Cu") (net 2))
 (segment (start 108.1 81.28) (end 107.465 81.915) (width 0.25) (layer "F.Cu") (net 2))
 (segment (start 122.7 82.55) (end 132.75 72.5) (width 0.25) (layer "F.Cu") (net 9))
 (segment (start 131.445 68.58) (end 130.75 69.275) (width 0.25) (layer "F.Cu") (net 9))
 (segment (start 109.07 82.55) (end 116.205 82.55) (width 0.25) (layer "F.Cu") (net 9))
 (segment (start 130.75 69.275) (end 130.75 70.25) (width 0.25) (layer "F.Cu") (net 9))
 (segment (start 116.205 82.55) (end 122.7 82.55) (width 0.25) (layer "F.Cu") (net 9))
 (via (at 130.75 70.25) (size 0.8) (drill 0.4) (layers "F.Cu" "B.Cu") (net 9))
 (via (at 132.75 72.5) (size 0.8) (drill 0.4) (layers "F.Cu" "B.Cu") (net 9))
 (segment (start 130.75 70.5) (end 130.75 70.25) (width 0.25) (layer "B.Cu") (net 9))
 (segment (start 132.75 72.5) (end 130.75 70.5) (width 0.25) (layer "B.Cu") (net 9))
 (segment (start 122.555 80.01) (end 133.985 68.58) (width 0.25) (layer "F.Cu") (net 3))
 (segment (start 109.07 80.01) (end 122.555 80.01) (width 0.25) (layer "F.Cu") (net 3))
 (segment (start 134.105 71) (end 136.525 68.58) (width 0.25) (layer "F.Cu") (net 1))
 (segment (start 109.07 81.28) (end 122.47 81.28) (width 0.25) (layer "F.Cu") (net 1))
 (segment (start 132.75 71) (end 134.105 71) (width 0.25) (layer "F.Cu") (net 1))
 (segment (start 122.47 81.28) (end 132.75 71) (width 0.25) (layer "F.Cu") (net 1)))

